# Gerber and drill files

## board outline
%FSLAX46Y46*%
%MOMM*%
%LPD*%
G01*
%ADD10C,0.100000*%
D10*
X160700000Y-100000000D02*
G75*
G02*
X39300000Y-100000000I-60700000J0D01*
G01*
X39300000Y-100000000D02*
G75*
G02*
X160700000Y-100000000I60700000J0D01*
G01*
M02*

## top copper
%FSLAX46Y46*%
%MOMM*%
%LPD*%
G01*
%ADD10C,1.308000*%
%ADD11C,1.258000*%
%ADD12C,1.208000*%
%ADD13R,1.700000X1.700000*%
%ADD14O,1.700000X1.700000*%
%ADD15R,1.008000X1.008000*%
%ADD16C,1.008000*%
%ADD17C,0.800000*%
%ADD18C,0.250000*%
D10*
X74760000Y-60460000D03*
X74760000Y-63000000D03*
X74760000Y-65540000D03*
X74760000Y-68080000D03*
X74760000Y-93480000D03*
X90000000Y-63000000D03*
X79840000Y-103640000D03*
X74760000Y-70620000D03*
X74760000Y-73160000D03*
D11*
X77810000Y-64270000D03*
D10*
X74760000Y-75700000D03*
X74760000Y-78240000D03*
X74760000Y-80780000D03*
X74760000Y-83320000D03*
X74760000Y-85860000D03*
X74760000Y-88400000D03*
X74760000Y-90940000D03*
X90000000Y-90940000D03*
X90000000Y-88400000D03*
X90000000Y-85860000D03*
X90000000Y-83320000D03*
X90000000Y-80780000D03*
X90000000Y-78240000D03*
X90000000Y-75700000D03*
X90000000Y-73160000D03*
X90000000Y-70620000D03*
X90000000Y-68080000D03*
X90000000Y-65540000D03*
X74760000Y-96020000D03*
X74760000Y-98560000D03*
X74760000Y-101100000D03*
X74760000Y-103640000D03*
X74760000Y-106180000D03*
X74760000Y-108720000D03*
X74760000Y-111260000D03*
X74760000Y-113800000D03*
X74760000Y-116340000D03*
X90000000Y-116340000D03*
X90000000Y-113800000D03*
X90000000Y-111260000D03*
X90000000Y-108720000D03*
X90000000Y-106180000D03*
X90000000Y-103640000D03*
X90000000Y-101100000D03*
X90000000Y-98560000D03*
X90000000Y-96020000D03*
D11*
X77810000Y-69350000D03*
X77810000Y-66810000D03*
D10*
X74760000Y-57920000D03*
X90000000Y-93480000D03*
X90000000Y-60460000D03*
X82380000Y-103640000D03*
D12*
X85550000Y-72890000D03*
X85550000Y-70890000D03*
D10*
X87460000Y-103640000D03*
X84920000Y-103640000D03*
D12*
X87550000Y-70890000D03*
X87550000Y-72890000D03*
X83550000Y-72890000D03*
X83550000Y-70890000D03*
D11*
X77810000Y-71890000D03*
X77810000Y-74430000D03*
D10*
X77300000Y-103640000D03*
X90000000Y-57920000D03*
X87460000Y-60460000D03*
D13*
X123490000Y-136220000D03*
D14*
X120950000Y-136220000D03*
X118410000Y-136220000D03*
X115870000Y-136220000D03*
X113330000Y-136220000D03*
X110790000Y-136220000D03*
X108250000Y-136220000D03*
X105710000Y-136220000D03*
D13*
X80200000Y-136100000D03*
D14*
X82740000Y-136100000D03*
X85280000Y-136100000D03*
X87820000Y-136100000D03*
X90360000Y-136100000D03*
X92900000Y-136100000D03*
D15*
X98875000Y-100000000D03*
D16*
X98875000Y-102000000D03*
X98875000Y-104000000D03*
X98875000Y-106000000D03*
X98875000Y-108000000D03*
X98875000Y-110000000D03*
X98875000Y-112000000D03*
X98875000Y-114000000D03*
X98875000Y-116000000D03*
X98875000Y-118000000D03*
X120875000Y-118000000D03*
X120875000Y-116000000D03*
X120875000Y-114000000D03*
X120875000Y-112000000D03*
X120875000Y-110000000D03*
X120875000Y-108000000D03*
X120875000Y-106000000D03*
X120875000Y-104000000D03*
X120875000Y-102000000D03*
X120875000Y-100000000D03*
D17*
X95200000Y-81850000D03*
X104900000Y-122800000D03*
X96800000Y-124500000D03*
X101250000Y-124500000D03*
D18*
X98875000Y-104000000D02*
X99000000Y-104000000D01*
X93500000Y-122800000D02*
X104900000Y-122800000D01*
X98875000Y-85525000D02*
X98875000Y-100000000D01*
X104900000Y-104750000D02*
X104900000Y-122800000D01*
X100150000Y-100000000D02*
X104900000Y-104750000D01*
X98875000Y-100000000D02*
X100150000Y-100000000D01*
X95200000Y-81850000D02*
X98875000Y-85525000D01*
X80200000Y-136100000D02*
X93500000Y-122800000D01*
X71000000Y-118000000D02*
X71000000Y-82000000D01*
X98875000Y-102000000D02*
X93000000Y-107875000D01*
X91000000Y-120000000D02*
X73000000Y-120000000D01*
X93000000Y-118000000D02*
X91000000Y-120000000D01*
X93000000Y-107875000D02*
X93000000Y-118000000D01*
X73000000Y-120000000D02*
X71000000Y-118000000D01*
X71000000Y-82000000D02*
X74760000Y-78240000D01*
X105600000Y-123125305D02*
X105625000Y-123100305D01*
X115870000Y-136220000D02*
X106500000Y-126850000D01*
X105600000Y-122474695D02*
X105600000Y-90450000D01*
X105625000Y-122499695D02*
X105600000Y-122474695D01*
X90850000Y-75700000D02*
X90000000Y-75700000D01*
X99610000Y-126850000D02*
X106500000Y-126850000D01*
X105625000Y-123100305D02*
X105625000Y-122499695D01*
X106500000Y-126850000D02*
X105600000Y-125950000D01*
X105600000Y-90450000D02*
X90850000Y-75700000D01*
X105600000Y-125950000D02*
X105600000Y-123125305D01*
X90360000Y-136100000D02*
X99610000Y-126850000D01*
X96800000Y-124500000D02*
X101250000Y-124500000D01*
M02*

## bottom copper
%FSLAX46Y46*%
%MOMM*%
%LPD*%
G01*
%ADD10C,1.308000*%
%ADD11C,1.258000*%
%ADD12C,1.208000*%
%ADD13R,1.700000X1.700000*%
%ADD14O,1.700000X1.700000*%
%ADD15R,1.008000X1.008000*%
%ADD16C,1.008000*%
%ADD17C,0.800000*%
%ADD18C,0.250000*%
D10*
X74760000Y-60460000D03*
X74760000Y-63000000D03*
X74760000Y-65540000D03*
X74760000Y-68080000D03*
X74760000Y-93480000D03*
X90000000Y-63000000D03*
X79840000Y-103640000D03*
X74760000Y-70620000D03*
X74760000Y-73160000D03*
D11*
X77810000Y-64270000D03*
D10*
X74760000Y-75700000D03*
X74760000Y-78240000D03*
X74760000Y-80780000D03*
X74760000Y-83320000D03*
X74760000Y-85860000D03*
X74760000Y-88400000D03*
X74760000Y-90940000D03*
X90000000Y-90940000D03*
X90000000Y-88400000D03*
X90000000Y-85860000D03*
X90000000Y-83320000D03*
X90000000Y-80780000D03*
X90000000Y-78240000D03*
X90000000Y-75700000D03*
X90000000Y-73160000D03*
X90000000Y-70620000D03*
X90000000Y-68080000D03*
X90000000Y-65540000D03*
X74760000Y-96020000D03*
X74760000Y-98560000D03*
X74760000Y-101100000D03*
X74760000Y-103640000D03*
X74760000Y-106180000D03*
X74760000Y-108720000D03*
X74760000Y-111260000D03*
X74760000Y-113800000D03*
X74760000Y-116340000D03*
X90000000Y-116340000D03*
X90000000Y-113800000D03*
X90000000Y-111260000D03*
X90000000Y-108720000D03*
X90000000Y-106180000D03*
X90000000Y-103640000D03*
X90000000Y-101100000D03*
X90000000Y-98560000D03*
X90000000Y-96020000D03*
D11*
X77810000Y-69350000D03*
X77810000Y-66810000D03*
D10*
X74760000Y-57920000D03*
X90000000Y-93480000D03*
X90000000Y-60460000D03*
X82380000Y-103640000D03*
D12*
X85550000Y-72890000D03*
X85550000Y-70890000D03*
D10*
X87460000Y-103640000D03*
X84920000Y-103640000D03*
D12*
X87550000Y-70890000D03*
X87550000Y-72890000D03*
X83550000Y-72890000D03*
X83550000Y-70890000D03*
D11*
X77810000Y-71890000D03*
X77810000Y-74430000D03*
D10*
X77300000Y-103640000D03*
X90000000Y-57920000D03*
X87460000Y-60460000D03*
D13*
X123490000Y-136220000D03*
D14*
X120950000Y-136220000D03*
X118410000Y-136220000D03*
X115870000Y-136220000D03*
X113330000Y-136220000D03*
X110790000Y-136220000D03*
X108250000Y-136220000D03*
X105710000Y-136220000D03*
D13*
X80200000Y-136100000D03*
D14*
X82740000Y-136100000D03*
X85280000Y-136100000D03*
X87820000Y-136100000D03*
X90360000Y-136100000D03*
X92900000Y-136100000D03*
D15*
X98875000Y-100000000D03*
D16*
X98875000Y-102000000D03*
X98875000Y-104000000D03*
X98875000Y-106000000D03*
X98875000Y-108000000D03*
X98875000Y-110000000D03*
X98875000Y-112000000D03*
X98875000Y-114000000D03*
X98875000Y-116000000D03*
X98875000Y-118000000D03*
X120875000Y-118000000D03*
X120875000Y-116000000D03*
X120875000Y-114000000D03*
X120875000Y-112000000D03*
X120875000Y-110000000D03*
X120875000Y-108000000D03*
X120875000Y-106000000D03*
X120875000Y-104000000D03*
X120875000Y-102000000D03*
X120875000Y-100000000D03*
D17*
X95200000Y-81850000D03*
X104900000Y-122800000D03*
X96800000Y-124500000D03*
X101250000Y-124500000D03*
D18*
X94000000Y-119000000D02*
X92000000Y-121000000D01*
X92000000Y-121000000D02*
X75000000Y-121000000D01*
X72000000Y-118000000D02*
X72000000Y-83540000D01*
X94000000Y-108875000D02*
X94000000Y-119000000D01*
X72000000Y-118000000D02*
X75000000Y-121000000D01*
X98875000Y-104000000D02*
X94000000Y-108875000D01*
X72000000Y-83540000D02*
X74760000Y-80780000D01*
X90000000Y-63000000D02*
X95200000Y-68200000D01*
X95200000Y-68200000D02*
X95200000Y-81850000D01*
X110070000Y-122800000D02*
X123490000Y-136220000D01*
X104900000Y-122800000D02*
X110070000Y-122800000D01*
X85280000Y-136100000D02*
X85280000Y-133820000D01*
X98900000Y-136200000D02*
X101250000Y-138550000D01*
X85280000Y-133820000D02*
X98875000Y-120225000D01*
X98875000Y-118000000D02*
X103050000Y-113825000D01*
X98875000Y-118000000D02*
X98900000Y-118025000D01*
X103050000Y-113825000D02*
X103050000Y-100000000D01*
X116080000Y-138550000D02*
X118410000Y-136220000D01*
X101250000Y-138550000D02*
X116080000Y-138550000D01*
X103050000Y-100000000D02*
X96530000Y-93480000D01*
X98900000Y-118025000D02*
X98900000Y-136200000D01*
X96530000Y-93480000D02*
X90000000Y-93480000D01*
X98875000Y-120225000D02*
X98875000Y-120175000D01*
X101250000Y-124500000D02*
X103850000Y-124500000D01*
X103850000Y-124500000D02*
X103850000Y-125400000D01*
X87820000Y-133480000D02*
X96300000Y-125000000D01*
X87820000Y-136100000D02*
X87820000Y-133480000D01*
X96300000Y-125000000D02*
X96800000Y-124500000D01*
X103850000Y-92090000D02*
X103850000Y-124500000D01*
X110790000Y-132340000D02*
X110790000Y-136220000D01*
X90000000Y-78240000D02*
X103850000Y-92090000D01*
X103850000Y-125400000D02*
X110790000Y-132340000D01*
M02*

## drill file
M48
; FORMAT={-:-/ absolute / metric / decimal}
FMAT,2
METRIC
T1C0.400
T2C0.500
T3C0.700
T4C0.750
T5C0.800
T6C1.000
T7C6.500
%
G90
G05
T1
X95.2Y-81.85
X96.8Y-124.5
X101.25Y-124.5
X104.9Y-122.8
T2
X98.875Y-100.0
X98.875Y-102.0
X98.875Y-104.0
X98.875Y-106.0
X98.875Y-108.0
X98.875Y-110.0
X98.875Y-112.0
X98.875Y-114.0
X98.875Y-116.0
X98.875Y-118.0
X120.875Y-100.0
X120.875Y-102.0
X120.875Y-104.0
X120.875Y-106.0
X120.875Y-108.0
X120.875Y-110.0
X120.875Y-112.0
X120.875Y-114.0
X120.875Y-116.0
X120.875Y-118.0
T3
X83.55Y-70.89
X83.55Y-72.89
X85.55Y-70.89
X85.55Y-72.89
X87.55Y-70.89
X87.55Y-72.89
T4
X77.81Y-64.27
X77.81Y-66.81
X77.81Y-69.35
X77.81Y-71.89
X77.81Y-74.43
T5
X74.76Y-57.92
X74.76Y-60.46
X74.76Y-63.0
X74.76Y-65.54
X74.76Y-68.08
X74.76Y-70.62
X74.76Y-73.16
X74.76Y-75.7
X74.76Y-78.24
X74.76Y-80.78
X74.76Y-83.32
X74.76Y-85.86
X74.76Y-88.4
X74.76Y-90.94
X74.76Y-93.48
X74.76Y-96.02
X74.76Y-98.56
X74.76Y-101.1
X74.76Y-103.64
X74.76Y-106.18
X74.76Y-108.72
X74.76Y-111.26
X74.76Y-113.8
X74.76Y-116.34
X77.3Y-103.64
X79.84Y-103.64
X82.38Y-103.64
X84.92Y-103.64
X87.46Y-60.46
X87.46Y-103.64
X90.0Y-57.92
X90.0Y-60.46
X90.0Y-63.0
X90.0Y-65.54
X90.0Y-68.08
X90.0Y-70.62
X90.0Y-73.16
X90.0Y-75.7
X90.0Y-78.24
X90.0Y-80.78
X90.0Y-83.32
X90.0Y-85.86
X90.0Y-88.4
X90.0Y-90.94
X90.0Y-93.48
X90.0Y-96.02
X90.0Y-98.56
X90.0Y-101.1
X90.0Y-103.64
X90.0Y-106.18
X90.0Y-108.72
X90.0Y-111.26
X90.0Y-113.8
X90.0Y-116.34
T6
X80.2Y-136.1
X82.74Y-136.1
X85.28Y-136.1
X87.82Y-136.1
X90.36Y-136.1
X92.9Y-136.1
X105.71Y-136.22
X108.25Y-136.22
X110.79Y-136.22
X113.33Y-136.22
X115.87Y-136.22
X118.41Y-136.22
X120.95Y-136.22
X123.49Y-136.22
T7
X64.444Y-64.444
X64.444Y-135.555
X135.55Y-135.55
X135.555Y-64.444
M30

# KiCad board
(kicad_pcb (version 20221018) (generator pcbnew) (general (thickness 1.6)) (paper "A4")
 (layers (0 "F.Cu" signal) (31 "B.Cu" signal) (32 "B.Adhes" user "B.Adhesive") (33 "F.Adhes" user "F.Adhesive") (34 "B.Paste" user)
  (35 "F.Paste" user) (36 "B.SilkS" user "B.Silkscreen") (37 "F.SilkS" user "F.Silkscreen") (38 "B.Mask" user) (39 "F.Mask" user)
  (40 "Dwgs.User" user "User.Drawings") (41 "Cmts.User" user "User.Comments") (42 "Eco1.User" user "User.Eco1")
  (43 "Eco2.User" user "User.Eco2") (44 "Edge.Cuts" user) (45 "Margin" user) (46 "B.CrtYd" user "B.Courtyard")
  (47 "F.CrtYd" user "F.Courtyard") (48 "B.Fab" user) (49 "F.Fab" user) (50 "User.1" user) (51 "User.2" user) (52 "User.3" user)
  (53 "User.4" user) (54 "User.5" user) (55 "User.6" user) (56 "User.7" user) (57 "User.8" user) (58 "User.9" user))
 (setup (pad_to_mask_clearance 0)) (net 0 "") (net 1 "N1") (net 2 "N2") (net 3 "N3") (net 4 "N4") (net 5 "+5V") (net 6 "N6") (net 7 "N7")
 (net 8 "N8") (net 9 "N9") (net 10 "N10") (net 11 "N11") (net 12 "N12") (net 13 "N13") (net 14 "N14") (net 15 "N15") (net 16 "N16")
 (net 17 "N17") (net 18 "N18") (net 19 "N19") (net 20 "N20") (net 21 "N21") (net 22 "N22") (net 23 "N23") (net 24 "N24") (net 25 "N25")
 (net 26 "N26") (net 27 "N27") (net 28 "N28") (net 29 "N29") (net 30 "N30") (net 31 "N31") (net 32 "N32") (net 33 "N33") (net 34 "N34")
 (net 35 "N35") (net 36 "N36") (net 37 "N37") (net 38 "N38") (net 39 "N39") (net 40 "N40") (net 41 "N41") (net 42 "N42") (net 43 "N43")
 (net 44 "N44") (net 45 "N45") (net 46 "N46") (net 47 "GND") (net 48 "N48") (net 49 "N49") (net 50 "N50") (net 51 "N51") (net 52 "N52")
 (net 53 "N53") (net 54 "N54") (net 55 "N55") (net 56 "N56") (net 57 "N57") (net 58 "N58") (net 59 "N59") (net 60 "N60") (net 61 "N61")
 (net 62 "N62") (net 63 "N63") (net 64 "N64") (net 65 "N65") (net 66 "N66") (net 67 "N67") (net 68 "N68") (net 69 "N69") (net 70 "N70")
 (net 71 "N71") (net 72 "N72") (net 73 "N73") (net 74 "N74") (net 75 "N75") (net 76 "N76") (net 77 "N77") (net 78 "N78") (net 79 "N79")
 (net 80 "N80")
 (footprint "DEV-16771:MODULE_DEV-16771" (layer "F.Cu") (at 82.38 87.13 -90)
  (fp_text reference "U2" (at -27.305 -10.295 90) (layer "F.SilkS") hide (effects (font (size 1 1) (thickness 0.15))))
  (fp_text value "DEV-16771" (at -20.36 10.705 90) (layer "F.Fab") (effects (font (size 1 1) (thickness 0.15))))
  (pad "0" thru_hole circle (at -26.67 7.62 270) (size 1.308 1.308) (drill 0.8) (layers "*.Cu" "*.Mask") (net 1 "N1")
   (solder_mask_margin 0.102))
  (pad "1" thru_hole circle (at -24.13 7.62 270) (size 1.308 1.308) (drill 0.8) (layers "*.Cu" "*.Mask") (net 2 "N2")
   (solder_mask_margin 0.102))
  (pad "2" thru_hole circle (at -21.59 7.62 270) (size 1.308 1.308) (drill 0.8) (layers "*.Cu" "*.Mask") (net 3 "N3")
   (solder_mask_margin 0.102))
  (pad "3" thru_hole circle (at -19.05 7.62 270) (size 1.308 1.308) (drill 0.8) (layers "*.Cu" "*.Mask") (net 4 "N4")
   (solder_mask_margin 0.102))
  (pad "3.3V_1" thru_hole circle (at 6.35 7.62 270) (size 1.308 1.308) (drill 0.8) (layers "*.Cu" "*.Mask") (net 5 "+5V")
   (solder_mask_margin 0.102))
  (pad "3.3V_2" thru_hole circle (at -24.13 -7.62 270) (size 1.308 1.308) (drill 0.8) (layers "*.Cu" "*.Mask") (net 5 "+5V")
   (solder_mask_margin 0.102))
  (pad "3.3V_3" thru_hole circle (at 16.51 2.54 270) (size 1.308 1.308) (drill 0.8) (layers "*.Cu" "*.Mask") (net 5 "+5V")
   (solder_mask_margin 0.102))
  (pad "4" thru_hole circle (at -16.51 7.62 270) (size 1.308 1.308) (drill 0.8) (layers "*.Cu" "*.Mask") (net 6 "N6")
   (solder_mask_margin 0.102))
  (pad "5" thru_hole circle (at -13.97 7.62 270) (size 1.308 1.308) (drill 0.8) (layers "*.Cu" "*.Mask") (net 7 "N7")
   (solder_mask_margin 0.102))
  (pad "5V" thru_hole circle (at -22.86 4.57 270) (size 1.258 1.258) (drill 0.75) (layers "*.Cu" "*.Mask") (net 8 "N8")
   (solder_mask_margin 0.102))
  (pad "6" thru_hole circle (at -11.43 7.62 270) (size 1.308 1.308) (drill 0.8) (layers "*.Cu" "*.Mask") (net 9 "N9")
   (solder_mask_margin 0.102))
  (pad "7" thru_hole circle (at -8.89 7.62 270) (size 1.308 1.308) (drill 0.8) (layers "*.Cu" "*.Mask") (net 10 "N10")
   (solder_mask_margin 0.102))
  (pad "8" thru_hole circle (at -6.35 7.62 270) (size 1.308 1.308) (drill 0.8) (layers "*.Cu" "*.Mask") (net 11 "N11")
   (solder_mask_margin 0.102))
  (pad "9" thru_hole circle (at -3.81 7.62 270) (size 1.308 1.308) (drill 0.8) (layers "*.Cu" "*.Mask") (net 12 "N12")
   (solder_mask_margin 0.102))
  (pad "10" thru_hole circle (at -1.27 7.62 270) (size 1.308 1.308) (drill 0.8) (layers "*.Cu" "*.Mask") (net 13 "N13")
   (solder_mask_margin 0.102))
  (pad "11" thru_hole circle (at 1.27 7.62 270) (size 1.308 1.308) (drill 0.8) (layers "*.Cu" "*.Mask") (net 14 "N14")
   (solder_mask_margin 0.102))
  (pad "12" thru_hole circle (at 3.81 7.62 270) (size 1.308 1.308) (drill 0.8) (layers "*.Cu" "*.Mask") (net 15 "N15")
   (solder_mask_margin 0.102))
  (pad "13" thru_hole circle (at 3.81 -7.62 270) (size 1.308 1.308) (drill 0.8) (layers "*.Cu" "*.Mask") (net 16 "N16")
   (solder_mask_margin 0.102))
  (pad "14" thru_hole circle (at 1.27 -7.62 270) (size 1.308 1.308) (drill 0.8) (layers "*.Cu" "*.Mask") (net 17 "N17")
   (solder_mask_margin 0.102))
  (pad "15" thru_hole circle (at -1.27 -7.62 270) (size 1.308 1.308) (drill 0.8) (layers "*.Cu" "*.Mask") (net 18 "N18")
   (solder_mask_margin 0.102))
  (pad "16" thru_hole circle (at -3.81 -7.62 270) (size 1.308 1.308) (drill 0.8) (layers "*.Cu" "*.Mask") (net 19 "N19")
   (solder_mask_margin 0.102))
  (pad "17" thru_hole circle (at -6.35 -7.62 270) (size 1.308 1.308) (drill 0.8) (layers "*.Cu" "*.Mask") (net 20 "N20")
   (solder_mask_margin 0.102))
  (pad "18" thru_hole circle (at -8.89 -7.62 270) (size 1.308 1.308) (drill 0.8) (layers "*.Cu" "*.Mask") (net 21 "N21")
   (solder_mask_margin 0.102))
  (pad "19" thru_hole circle (at -11.43 -7.62 270) (size 1.308 1.308) (drill 0.8) (layers "*.Cu" "*.Mask") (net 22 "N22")
   (solder_mask_margin 0.102))
  (pad "20" thru_hole circle (at -13.97 -7.62 270) (size 1.308 1.308) (drill 0.8) (layers "*.Cu" "*.Mask") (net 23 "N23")
   (solder_mask_margin 0.102))
  (pad "21" thru_hole circle (at -16.51 -7.62 270) (size 1.308 1.308) (drill 0.8) (layers "*.Cu" "*.Mask") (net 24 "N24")
   (solder_mask_margin 0.102))
  (pad "22" thru_hole circle (at -19.05 -7.62 270) (size 1.308 1.308) (drill 0.8) (layers "*.Cu" "*.Mask") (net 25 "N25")
   (solder_mask_margin 0.102))
  (pad "23" thru_hole circle (at -21.59 -7.62 270) (size 1.308 1.308) (drill 0.8) (layers "*.Cu" "*.Mask") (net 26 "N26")
   (solder_mask_margin 0.102))
  (pad "24" thru_hole circle (at 8.89 7.62 270) (size 1.308 1.308) (drill 0.8) (layers "*.Cu" "*.Mask") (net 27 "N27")
   (solder_mask_margin 0.102))
  (pad "25" thru_hole circle (at 11.43 7.62 270) (size 1.308 1.308) (drill 0.8) (layers "*.Cu" "*.Mask") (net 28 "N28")
   (solder_mask_margin 0.102))
  (pad "26" thru_hole circle (at 13.97 7.62 270) (size 1.308 1.308) (drill 0.8) (layers "*.Cu" "*.Mask") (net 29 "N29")
   (solder_mask_margin 0.102))
  (pad "27" thru_hole circle (at 16.51 7.62 270) (size 1.308 1.308) (drill 0.8) (layers "*.Cu" "*.Mask") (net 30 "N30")
   (solder_mask_margin 0.102))
  (pad "28" thru_hole circle (at 19.05 7.62 270) (size 1.308 1.308) (drill 0.8) (layers "*.Cu" "*.Mask") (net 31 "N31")
   (solder_mask_margin 0.102))
  (pad "29" thru_hole circle (at 21.59 7.62 270) (size 1.308 1.308) (drill 0.8) (layers "*.Cu" "*.Mask") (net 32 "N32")
   (solder_mask_margin 0.102))
  (pad "30" thru_hole circle (at 24.13 7.62 270) (size 1.308 1.308) (drill 0.8) (layers "*.Cu" "*.Mask") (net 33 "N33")
   (solder_mask_margin 0.102))
  (pad "31" thru_hole circle (at 26.67 7.62 270) (size 1.308 1.308) (drill 0.8) (layers "*.Cu" "*.Mask") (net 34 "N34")
   (solder_mask_margin 0.102))
  (pad "32" thru_hole circle (at 29.21 7.62 270) (size 1.308 1.308) (drill 0.8) (layers "*.Cu" "*.Mask") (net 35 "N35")
   (solder_mask_margin 0.102))
  (pad "33" thru_hole circle (at 29.21 -7.62 270) (size 1.308 1.308) (drill 0.8) (layers "*.Cu" "*.Mask") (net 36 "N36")
   (solder_mask_margin 0.102))
  (pad "34" thru_hole circle (at 26.67 -7.62 270) (size 1.308 1.308) (drill 0.8) (layers "*.Cu" "*.Mask") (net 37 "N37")
   (solder_mask_margin 0.102))
  (pad "35" thru_hole circle (at 24.13 -7.62 270) (size 1.308 1.308) (drill 0.8) (layers "*.Cu" "*.Mask") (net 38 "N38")
   (solder_mask_margin 0.102))
  (pad "36" thru_hole circle (at 21.59 -7.62 270) (size 1.308 1.308) (drill 0.8) (layers "*.Cu" "*.Mask") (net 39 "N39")
   (solder_mask_margin 0.102))
  (pad "37" thru_hole circle (at 19.05 -7.62 270) (size 1.308 1.308) (drill 0.8) (layers "*.Cu" "*.Mask") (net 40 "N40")
   (solder_mask_margin 0.102))
  (pad "38" thru_hole circle (at 16.51 -7.62 270) (size 1.308 1.308) (drill 0.8) (layers "*.Cu" "*.Mask") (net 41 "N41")
   (solder_mask_margin 0.102))
  (pad "39" thru_hole circle (at 13.97 -7.62 270) (size 1.308 1.308) (drill 0.8) (layers "*.Cu" "*.Mask") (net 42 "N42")
   (solder_mask_margin 0.102))
  (pad "40" thru_hole circle (at 11.43 -7.62 270) (size 1.308 1.308) (drill 0.8) (layers "*.Cu" "*.Mask") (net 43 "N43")
   (solder_mask_margin 0.102))
  (pad "41" thru_hole circle (at 8.89 -7.62 270) (size 1.308 1.308) (drill 0.8) (layers "*.Cu" "*.Mask") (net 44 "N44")
   (solder_mask_margin 0.102))
  (pad "D+" thru_hole circle (at -17.78 4.57 270) (size 1.258 1.258) (drill 0.75) (layers "*.Cu" "*.Mask") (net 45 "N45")
   (solder_mask_margin 0.102))
  (pad "D-" thru_hole circle (at -20.32 4.57 270) (size 1.258 1.258) (drill 0.75) (layers "*.Cu" "*.Mask") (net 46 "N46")
   (solder_mask_margin 0.102))
  (pad "GND1" thru_hole circle (at -29.21 7.62 270) (size 1.308 1.308) (drill 0.8) (layers "*.Cu" "*.Mask") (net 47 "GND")
   (solder_mask_margin 0.102))
  (pad "GND2" thru_hole circle (at 6.35 -7.62 270) (size 1.308 1.308) (drill 0.8) (layers "*.Cu" "*.Mask") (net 47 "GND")
   (solder_mask_margin 0.102))
  (pad "GND3" thru_hole circle (at -26.67 -7.62 270) (size 1.308 1.308) (drill 0.8) (layers "*.Cu" "*.Mask") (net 47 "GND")
   (solder_mask_margin 0.102))
  (pad "GND4" thru_hole circle (at 16.51 0 270) (size 1.308 1.308) (drill 0.8) (layers "*.Cu" "*.Mask") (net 47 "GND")
   (solder_mask_margin 0.102))
  (pad "GND5" thru_hole circle (at -14.24 -3.17 270) (size 1.208 1.208) (drill 0.7) (layers "*.Cu" "*.Mask") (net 47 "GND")
   (solder_mask_margin 0.102))
  (pad "LED" thru_hole circle (at -16.24 -3.17 270) (size 1.208 1.208) (drill 0.7) (layers "*.Cu" "*.Mask") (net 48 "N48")
   (solder_mask_margin 0.102))
  (pad "ON/OFF" thru_hole circle (at 16.51 -5.08 270) (size 1.308 1.308) (drill 0.8) (layers "*.Cu" "*.Mask") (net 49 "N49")
   (solder_mask_margin 0.102))
  (pad "PROGRAM" thru_hole circle (at 16.51 -2.54 270) (size 1.308 1.308) (drill 0.8) (layers "*.Cu" "*.Mask") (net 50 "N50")
   (solder_mask_margin 0.102))
  (pad "R+" thru_hole circle (at -16.24 -5.17 270) (size 1.208 1.208) (drill 0.7) (layers "*.Cu" "*.Mask") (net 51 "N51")
   (solder_mask_margin 0.102))
  (pad "R-" thru_hole circle (at -14.24 -5.17 270) (size 1.208 1.208) (drill 0.7) (layers "*.Cu" "*.Mask") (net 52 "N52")
   (solder_mask_margin 0.102))
  (pad "T+" thru_hole circle (at -14.24 -1.17 270) (size 1.208 1.208) (drill 0.7) (layers "*.Cu" "*.Mask") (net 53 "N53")
   (solder_mask_margin 0.102))
  (pad "T-" thru_hole circle (at -16.24 -1.17 270) (size 1.208 1.208) (drill 0.7) (layers "*.Cu" "*.Mask") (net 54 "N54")
   (solder_mask_margin 0.102))
  (pad "USB_GND1" thru_hole circle (at -15.24 4.57 270) (size 1.258 1.258) (drill 0.75) (layers "*.Cu" "*.Mask") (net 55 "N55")
   (solder_mask_margin 0.102))
  (pad "USB_GND2" thru_hole circle (at -12.7 4.57 270) (size 1.258 1.258) (drill 0.75) (layers "*.Cu" "*.Mask") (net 55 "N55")
   (solder_mask_margin 0.102))
  (pad "VBAT" thru_hole circle (at 16.51 5.08 270) (size 1.308 1.308) (drill 0.8) (layers "*.Cu" "*.Mask") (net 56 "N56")
   (solder_mask_margin 0.102))
  (pad "VIN" thru_hole circle (at -29.21 -7.62 270) (size 1.308 1.308) (drill 0.8) (layers "*.Cu" "*.Mask") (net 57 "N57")
   (solder_mask_margin 0.102))
  (pad "VUSB" thru_hole circle (at -26.67 -5.08 270) (size 1.308 1.308) (drill 0.8) (layers "*.Cu" "*.Mask") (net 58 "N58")
   (solder_mask_margin 0.102)))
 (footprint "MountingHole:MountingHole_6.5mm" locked (layer "F.Cu") (at 64.4445 135.555)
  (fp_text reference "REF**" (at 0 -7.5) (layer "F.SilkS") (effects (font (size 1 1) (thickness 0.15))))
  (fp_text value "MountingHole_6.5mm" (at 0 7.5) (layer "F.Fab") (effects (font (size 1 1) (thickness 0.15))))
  (pad "" np_thru_hole circle locked (at 0 0) (size 6.5 6.5) (drill 6.5) (layers "F&B.Cu" "*.Mask")))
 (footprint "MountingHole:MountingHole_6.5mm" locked (layer "F.Cu") (at 135.55 135.55)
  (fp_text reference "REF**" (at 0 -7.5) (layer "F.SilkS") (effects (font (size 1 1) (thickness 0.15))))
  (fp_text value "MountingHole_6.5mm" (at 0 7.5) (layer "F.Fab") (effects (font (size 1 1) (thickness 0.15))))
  (pad "" np_thru_hole circle locked (at 0 0) (size 6.5 6.5) (drill 6.5) (layers "F&B.Cu" "*.Mask")))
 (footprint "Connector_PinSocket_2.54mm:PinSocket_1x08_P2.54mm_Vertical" (layer "F.Cu") (at 123.49 136.22 -90)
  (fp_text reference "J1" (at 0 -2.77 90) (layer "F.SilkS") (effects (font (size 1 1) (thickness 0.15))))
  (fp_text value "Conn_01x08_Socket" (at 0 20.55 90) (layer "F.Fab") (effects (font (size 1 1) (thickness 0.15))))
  (pad "1" thru_hole rect (at 0 0 270) (size 1.7 1.7) (drill 1) (layers "*.Cu" "*.Mask") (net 5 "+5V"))
  (pad "2" thru_hole oval (at 0 2.54 270) (size 1.7 1.7) (drill 1) (layers "*.Cu" "*.Mask") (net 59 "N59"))
  (pad "3" thru_hole oval (at 0 5.08 270) (size 1.7 1.7) (drill 1) (layers "*.Cu" "*.Mask") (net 47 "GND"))
  (pad "4" thru_hole oval (at 0 7.62 270) (size 1.7 1.7) (drill 1) (layers "*.Cu" "*.Mask") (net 22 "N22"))
  (pad "5" thru_hole oval (at 0 10.16 270) (size 1.7 1.7) (drill 1) (layers "*.Cu" "*.Mask") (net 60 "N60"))
  (pad "6" thru_hole oval (at 0 12.7 270) (size 1.7 1.7) (drill 1) (layers "*.Cu" "*.Mask") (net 21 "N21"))
  (pad "7" thru_hole oval (at 0 15.24 270) (size 1.7 1.7) (drill 1) (layers "*.Cu" "*.Mask") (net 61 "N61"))
  (pad "8" thru_hole oval (at 0 17.78 270) (size 1.7 1.7) (drill 1) (layers "*.Cu" "*.Mask") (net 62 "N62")))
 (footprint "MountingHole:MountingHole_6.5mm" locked (layer "F.Cu") (at 64.4445 64.4445)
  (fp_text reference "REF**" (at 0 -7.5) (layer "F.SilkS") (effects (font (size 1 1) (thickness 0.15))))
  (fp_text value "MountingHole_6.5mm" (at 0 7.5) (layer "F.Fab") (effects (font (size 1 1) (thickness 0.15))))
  (pad "" np_thru_hole circle locked (at 0 0) (size 6.5 6.5) (drill 6.5) (layers "F&B.Cu" "*.Mask")))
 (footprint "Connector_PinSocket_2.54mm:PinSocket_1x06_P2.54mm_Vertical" (layer "F.Cu") (at 80.2 136.1 90)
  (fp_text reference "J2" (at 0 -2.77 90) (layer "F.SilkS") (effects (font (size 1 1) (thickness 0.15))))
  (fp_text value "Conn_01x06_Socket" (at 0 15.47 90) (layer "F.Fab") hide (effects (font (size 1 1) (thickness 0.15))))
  (pad "1" thru_hole rect (at 0 0 90) (size 1.7 1.7) (drill 1) (layers "*.Cu" "*.Mask") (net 5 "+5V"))
  (pad "2" thru_hole oval (at 0 2.54 90) (size 1.7 1.7) (drill 1) (layers "*.Cu" "*.Mask") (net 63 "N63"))
  (pad "3" thru_hole oval (at 0 5.08 90) (size 1.7 1.7) (drill 1) (layers "*.Cu" "*.Mask") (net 47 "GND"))
  (pad "4" thru_hole oval (at 0 7.62 90) (size 1.7 1.7) (drill 1) (layers "*.Cu" "*.Mask") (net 21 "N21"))
  (pad "5" thru_hole oval (at 0 10.16 90) (size 1.7 1.7) (drill 1) (layers "*.Cu" "*.Mask") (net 22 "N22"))
  (pad "6" thru_hole oval (at 0 12.7 90) (size 1.7 1.7) (drill 1) (layers "*.Cu" "*.Mask") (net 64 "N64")))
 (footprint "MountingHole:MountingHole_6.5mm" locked (layer "F.Cu") (at 135.555 64.4445)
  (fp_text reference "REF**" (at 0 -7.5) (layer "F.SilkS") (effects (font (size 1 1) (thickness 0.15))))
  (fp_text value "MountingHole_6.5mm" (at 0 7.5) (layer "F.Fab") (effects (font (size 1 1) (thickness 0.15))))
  (pad "" np_thru_hole circle locked (at 0 0) (size 6.5 6.5) (drill 6.5) (layers "F&B.Cu" "*.Mask")))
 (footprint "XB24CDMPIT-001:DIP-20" (layer "F.Cu") (at 109.813 112.118)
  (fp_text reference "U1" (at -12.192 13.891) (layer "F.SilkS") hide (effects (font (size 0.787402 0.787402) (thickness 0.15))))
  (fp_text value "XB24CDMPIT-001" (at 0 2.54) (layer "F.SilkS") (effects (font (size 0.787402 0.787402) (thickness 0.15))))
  (pad "1" thru_hole rect (at -10.938 -12.118) (size 1.008 1.008) (drill 0.5) (layers "*.Cu" "*.Mask") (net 5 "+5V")
   (solder_mask_margin 0.102))
  (pad "2" thru_hole circle (at -10.938 -10.118) (size 1.008 1.008) (drill 0.5) (layers "*.Cu" "*.Mask") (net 10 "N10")
   (solder_mask_margin 0.102))
  (pad "3" thru_hole circle (at -10.938 -8.118) (size 1.008 1.008) (drill 0.5) (layers "*.Cu" "*.Mask") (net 11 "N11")
   (solder_mask_margin 0.102))
  (pad "4" thru_hole circle (at -10.938 -6.118) (size 1.008 1.008) (drill 0.5) (layers "*.Cu" "*.Mask") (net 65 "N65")
   (solder_mask_margin 0.102))
  (pad "5" thru_hole circle (at -10.938 -4.118) (size 1.008 1.008) (drill 0.5) (layers "*.Cu" "*.Mask") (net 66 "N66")
   (solder_mask_margin 0.102))
  (pad "6" thru_hole circle (at -10.938 -2.118) (size 1.008 1.008) (drill 0.5) (layers "*.Cu" "*.Mask") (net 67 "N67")
   (solder_mask_margin 0.102))
  (pad "7" thru_hole circle (at -10.938 -0.118) (size 1.008 1.008) (drill 0.5) (layers "*.Cu" "*.Mask") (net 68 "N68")
   (solder_mask_margin 0.102))
  (pad "8" thru_hole circle (at -10.938 1.882) (size 1.008 1.008) (drill 0.5) (layers "*.Cu" "*.Mask") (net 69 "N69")
   (solder_mask_margin 0.102))
  (pad "9" thru_hole circle (at -10.938 3.882) (size 1.008 1.008) (drill 0.5) (layers "*.Cu" "*.Mask") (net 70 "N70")
   (solder_mask_margin 0.102))
  (pad "10" thru_hole circle (at -10.938 5.882) (size 1.008 1.008) (drill 0.5) (layers "*.Cu" "*.Mask") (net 47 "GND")
   (solder_mask_margin 0.102))
  (pad "11" thru_hole circle (at 11.062 5.882) (size 1.008 1.008) (drill 0.5) (layers "*.Cu" "*.Mask") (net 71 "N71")
   (solder_mask_margin 0.102))
  (pad "12" thru_hole circle (at 11.062 3.882) (size 1.008 1.008) (drill 0.5) (layers "*.Cu" "*.Mask") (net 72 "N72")
   (solder_mask_margin 0.102))
  (pad "13" thru_hole circle (at 11.062 1.882) (size 1.008 1.008) (drill 0.5) (layers "*.Cu" "*.Mask") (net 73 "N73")
   (solder_mask_margin 0.102))
  (pad "14" thru_hole circle (at 11.062 -0.118) (size 1.008 1.008) (drill 0.5) (layers "*.Cu" "*.Mask") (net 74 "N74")
   (solder_mask_margin 0.102))
  (pad "15" thru_hole circle (at 11.062 -2.118) (size 1.008 1.008) (drill 0.5) (layers "*.Cu" "*.Mask") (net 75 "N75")
   (solder_mask_margin 0.102))
  (pad "16" thru_hole circle (at 11.062 -4.118) (size 1.008 1.008) (drill 0.5) (layers "*.Cu" "*.Mask") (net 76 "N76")
   (solder_mask_margin 0.102))
  (pad "17" thru_hole circle (at 11.062 -6.118) (size 1.008 1.008) (drill 0.5) (layers "*.Cu" "*.Mask") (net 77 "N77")
   (solder_mask_margin 0.102))
  (pad "18" thru_hole circle (at 11.062 -8.118) (size 1.008 1.008) (drill 0.5) (layers "*.Cu" "*.Mask") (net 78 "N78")
   (solder_mask_margin 0.102))
  (pad "19" thru_hole circle (at 11.062 -10.118) (size 1.008 1.008) (drill 0.5) (layers "*.Cu" "*.Mask") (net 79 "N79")
   (solder_mask_margin 0.102))
  (pad "20" thru_hole circle (at 11.062 -12.118) (size 1.008 1.008) (drill 0.5) (layers "*.Cu" "*.Mask") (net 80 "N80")
   (solder_mask_margin 0.102)))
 (gr_circle locked (center 100 100) (end 160.7 100) (stroke (width 0.1) (type solid)) (fill none) (layer "Edge.Cuts"))
 (segment (start 98.875 104) (end 99 104) (width 0.25) (layer "F.Cu") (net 11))
 (segment (start 94 119) (end 92 121) (width 0.25) (layer "B.Cu") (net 11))
 (segment (start 92 121) (end 75 121) (width 0.25) (layer "B.Cu") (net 11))
 (segment (start 72 118) (end 72 83.54) (width 0.25) (layer "B.Cu") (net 11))
 (segment (start 94 108.875) (end 94 119) (width 0.25) (layer "B.Cu") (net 11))
 (segment (start 72 118) (end 75 121) (width 0.25) (layer "B.Cu") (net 11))
 (segment (start 98.875 104) (end 94 108.875) (width 0.25) (layer "B.Cu") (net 11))
 (segment (start 72 83.54) (end 74.76 80.78) (width 0.25) (layer "B.Cu") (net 11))
 (segment (start 93.5 122.8) (end 104.9 122.8) (width 0.25) (layer "F.Cu") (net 5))
 (segment (start 98.875 85.525) (end 98.875 100) (width 0.25) (layer "F.Cu") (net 5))
 (segment (start 104.9 104.75) (end 104.9 122.8) (width 0.25) (layer "F.Cu") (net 5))
 (segment (start 100.15 100) (end 104.9 104.75) (width 0.25) (layer "F.Cu") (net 5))
 (segment (start 98.875 100) (end 100.15 100) (width 0.25) (layer "F.Cu") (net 5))
 (segment (start 95.2 81.85) (end 98.875 85.525) (width 0.25) (layer "F.Cu") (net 5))
 (segment (start 80.2 136.1) (end 93.5 122.8) (width 0.25) (layer "F.Cu") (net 5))
 (via (at 95.2 81.85) (size 0.8) (drill 0.4) (layers "F.Cu" "B.Cu") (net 5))
 (via (at 104.9 122.8) (size 0.8) (drill 0.4) (layers "F.Cu" "B.Cu") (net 5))
 (segment (start 90 63) (end 95.2 68.2) (width 0.25) (layer "B.Cu") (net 5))
 (segment (start 95.2 68.2) (end 95.2 81.85) (width 0.25) (layer "B.Cu") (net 5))
 (segment (start 110.07 122.8) (end 123.49 136.22) (width 0.25) (layer "B.Cu") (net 5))
 (segment (start 104.9 122.8) (end 110.07 122.8) (width 0.25) (layer "B.Cu") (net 5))
 (segment (start 71 118) (end 71 82) (width 0.25) (layer "F.Cu") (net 10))
 (segment (start 98.875 102) (end 93 107.875) (width 0.25) (layer "F.Cu") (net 10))
 (segment (start 91 120) (end 73 120) (width 0.25) (layer "F.Cu") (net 10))
 (segment (start 93 118) (end 91 120) (width 0.25) (layer "F.Cu") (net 10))
 (segment (start 93 107.875) (end 93 118) (width 0.25) (layer "F.Cu") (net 10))
 (segment (start 73 120) (end 71 118) (width 0.25) (layer "F.Cu") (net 10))
 (segment (start 71 82) (end 74.76 78.24) (width 0.25) (layer "F.Cu") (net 10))
 (segment (start 85.28 136.1) (end 85.28 133.82) (width 0.25) (layer "B.Cu") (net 47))
 (segment (start 98.9 136.2) (end 101.25 138.55) (width 0.25) (layer "B.Cu") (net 47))
 (segment (start 85.28 133.82) (end 98.875 120.225) (width 0.25) (layer "B.Cu") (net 47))
 (segment (start 98.875 118) (end 103.05 113.825) (width 0.25) (layer "B.Cu") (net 47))
 (segment (start 98.875 118) (end 98.9 118.025) (width 0.25) (layer "B.Cu") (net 47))
 (segment (start 103.05 113.825) (end 103.05 100) (width 0.25) (layer "B.Cu") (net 47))
 (segment (start 116.08 138.55) (end 118.41 136.22) (width 0.25) (layer "B.Cu") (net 47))
 (segment (start 101.25 138.55) (end 116.08 138.55) (width 0.25) (layer "B.Cu") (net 47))
 (segment (start 103.05 100) (end 96.53 93.48) (width 0.25) (layer "B.Cu") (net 47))
 (segment (start 98.9 118.025) (end 98.9 136.2) (width 0.25) (layer "B.Cu") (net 47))
 (segment (start 96.53 93.48) (end 90 93.48) (width 0.25) (layer "B.Cu") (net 47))
 (segment (start 98.875 120.225) (end 98.875 120.175) (width 0.25) (layer "B.Cu") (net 47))
 (segment (start 105.6 123.125305) (end 105.625 123.100305) (width 0.25) (layer "F.Cu") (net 22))
 (segment (start 115.87 136.22) (end 106.5 126.85) (width 0.25) (layer "F.Cu") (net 22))
 (segment (start 105.6 122.474695) (end 105.6 90.45) (width 0.25) (layer "F.Cu") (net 22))
 (segment (start 105.625 122.499695) (end 105.6 122.474695) (width 0.25) (layer "F.Cu") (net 22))
 (segment (start 90.85 75.7) (end 90 75.7) (width 0.25) (layer "F.Cu") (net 22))
 (segment (start 99.61 126.85) (end 106.5 126.85) (width 0.25) (layer "F.Cu") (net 22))
 (segment (start 105.625 123.100305) (end 105.625 122.499695) (width 0.25) (layer "F.Cu") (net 22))
 (segment (start 106.5 126.85) (end 105.6 125.95) (width 0.25) (layer "F.Cu") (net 22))
 (segment (start 105.6 90.45) (end 90.85 75.7) (width 0.25) (layer "F.Cu") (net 22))
 (segment (start 105.6 125.95) (end 105.6 123.125305) (width 0.25) (layer "F.Cu") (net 22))
 (segment (start 90.36 136.1) (end 99.61 126.85) (width 0.25) (layer "F.Cu") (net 22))
 (segment (start 96.8 124.5) (end 101.25 124.5) (width 0.25) (layer "F.Cu") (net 21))
 (via (at 96.8 124.5) (size 0.8) (drill 0.4) (layers "F.Cu" "B.Cu") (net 21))
 (via (at 101.25 124.5) (size 0.8) (drill 0.4) (layers "F.Cu" "B.Cu") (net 21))
 (segment (start 101.25 124.5) (end 103.85 124.5) (width 0.25) (layer "B.Cu") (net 21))
 (segment (start 103.85 124.5) (end 103.85 125.4) (width 0.25) (layer "B.Cu") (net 21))
 (segment (start 87.82 133.48) (end 96.3 125) (width 0.25) (layer "B.Cu") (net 21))
 (segment (start 87.82 136.1) (end 87.82 133.48) (width 0.25) (layer "B.Cu") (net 21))
 (segment (start 96.3 125) (end 96.8 124.5) (width 0.25) (layer "B.Cu") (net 21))
 (segment (start 103.85 92.09) (end 103.85 124.5) (width 0.25) (layer "B.Cu") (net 21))
 (segment (start 110.79 132.34) (end 110.79 136.22) (width 0.25) (layer "B.Cu") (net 21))
 (segment (start 90 78.24) (end 103.85 92.09) (width 0.25) (layer "B.Cu") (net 21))
 (segment (start 103.85 125.4) (end 110.79 132.34) (width 0.25) (layer "B.Cu") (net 21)))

